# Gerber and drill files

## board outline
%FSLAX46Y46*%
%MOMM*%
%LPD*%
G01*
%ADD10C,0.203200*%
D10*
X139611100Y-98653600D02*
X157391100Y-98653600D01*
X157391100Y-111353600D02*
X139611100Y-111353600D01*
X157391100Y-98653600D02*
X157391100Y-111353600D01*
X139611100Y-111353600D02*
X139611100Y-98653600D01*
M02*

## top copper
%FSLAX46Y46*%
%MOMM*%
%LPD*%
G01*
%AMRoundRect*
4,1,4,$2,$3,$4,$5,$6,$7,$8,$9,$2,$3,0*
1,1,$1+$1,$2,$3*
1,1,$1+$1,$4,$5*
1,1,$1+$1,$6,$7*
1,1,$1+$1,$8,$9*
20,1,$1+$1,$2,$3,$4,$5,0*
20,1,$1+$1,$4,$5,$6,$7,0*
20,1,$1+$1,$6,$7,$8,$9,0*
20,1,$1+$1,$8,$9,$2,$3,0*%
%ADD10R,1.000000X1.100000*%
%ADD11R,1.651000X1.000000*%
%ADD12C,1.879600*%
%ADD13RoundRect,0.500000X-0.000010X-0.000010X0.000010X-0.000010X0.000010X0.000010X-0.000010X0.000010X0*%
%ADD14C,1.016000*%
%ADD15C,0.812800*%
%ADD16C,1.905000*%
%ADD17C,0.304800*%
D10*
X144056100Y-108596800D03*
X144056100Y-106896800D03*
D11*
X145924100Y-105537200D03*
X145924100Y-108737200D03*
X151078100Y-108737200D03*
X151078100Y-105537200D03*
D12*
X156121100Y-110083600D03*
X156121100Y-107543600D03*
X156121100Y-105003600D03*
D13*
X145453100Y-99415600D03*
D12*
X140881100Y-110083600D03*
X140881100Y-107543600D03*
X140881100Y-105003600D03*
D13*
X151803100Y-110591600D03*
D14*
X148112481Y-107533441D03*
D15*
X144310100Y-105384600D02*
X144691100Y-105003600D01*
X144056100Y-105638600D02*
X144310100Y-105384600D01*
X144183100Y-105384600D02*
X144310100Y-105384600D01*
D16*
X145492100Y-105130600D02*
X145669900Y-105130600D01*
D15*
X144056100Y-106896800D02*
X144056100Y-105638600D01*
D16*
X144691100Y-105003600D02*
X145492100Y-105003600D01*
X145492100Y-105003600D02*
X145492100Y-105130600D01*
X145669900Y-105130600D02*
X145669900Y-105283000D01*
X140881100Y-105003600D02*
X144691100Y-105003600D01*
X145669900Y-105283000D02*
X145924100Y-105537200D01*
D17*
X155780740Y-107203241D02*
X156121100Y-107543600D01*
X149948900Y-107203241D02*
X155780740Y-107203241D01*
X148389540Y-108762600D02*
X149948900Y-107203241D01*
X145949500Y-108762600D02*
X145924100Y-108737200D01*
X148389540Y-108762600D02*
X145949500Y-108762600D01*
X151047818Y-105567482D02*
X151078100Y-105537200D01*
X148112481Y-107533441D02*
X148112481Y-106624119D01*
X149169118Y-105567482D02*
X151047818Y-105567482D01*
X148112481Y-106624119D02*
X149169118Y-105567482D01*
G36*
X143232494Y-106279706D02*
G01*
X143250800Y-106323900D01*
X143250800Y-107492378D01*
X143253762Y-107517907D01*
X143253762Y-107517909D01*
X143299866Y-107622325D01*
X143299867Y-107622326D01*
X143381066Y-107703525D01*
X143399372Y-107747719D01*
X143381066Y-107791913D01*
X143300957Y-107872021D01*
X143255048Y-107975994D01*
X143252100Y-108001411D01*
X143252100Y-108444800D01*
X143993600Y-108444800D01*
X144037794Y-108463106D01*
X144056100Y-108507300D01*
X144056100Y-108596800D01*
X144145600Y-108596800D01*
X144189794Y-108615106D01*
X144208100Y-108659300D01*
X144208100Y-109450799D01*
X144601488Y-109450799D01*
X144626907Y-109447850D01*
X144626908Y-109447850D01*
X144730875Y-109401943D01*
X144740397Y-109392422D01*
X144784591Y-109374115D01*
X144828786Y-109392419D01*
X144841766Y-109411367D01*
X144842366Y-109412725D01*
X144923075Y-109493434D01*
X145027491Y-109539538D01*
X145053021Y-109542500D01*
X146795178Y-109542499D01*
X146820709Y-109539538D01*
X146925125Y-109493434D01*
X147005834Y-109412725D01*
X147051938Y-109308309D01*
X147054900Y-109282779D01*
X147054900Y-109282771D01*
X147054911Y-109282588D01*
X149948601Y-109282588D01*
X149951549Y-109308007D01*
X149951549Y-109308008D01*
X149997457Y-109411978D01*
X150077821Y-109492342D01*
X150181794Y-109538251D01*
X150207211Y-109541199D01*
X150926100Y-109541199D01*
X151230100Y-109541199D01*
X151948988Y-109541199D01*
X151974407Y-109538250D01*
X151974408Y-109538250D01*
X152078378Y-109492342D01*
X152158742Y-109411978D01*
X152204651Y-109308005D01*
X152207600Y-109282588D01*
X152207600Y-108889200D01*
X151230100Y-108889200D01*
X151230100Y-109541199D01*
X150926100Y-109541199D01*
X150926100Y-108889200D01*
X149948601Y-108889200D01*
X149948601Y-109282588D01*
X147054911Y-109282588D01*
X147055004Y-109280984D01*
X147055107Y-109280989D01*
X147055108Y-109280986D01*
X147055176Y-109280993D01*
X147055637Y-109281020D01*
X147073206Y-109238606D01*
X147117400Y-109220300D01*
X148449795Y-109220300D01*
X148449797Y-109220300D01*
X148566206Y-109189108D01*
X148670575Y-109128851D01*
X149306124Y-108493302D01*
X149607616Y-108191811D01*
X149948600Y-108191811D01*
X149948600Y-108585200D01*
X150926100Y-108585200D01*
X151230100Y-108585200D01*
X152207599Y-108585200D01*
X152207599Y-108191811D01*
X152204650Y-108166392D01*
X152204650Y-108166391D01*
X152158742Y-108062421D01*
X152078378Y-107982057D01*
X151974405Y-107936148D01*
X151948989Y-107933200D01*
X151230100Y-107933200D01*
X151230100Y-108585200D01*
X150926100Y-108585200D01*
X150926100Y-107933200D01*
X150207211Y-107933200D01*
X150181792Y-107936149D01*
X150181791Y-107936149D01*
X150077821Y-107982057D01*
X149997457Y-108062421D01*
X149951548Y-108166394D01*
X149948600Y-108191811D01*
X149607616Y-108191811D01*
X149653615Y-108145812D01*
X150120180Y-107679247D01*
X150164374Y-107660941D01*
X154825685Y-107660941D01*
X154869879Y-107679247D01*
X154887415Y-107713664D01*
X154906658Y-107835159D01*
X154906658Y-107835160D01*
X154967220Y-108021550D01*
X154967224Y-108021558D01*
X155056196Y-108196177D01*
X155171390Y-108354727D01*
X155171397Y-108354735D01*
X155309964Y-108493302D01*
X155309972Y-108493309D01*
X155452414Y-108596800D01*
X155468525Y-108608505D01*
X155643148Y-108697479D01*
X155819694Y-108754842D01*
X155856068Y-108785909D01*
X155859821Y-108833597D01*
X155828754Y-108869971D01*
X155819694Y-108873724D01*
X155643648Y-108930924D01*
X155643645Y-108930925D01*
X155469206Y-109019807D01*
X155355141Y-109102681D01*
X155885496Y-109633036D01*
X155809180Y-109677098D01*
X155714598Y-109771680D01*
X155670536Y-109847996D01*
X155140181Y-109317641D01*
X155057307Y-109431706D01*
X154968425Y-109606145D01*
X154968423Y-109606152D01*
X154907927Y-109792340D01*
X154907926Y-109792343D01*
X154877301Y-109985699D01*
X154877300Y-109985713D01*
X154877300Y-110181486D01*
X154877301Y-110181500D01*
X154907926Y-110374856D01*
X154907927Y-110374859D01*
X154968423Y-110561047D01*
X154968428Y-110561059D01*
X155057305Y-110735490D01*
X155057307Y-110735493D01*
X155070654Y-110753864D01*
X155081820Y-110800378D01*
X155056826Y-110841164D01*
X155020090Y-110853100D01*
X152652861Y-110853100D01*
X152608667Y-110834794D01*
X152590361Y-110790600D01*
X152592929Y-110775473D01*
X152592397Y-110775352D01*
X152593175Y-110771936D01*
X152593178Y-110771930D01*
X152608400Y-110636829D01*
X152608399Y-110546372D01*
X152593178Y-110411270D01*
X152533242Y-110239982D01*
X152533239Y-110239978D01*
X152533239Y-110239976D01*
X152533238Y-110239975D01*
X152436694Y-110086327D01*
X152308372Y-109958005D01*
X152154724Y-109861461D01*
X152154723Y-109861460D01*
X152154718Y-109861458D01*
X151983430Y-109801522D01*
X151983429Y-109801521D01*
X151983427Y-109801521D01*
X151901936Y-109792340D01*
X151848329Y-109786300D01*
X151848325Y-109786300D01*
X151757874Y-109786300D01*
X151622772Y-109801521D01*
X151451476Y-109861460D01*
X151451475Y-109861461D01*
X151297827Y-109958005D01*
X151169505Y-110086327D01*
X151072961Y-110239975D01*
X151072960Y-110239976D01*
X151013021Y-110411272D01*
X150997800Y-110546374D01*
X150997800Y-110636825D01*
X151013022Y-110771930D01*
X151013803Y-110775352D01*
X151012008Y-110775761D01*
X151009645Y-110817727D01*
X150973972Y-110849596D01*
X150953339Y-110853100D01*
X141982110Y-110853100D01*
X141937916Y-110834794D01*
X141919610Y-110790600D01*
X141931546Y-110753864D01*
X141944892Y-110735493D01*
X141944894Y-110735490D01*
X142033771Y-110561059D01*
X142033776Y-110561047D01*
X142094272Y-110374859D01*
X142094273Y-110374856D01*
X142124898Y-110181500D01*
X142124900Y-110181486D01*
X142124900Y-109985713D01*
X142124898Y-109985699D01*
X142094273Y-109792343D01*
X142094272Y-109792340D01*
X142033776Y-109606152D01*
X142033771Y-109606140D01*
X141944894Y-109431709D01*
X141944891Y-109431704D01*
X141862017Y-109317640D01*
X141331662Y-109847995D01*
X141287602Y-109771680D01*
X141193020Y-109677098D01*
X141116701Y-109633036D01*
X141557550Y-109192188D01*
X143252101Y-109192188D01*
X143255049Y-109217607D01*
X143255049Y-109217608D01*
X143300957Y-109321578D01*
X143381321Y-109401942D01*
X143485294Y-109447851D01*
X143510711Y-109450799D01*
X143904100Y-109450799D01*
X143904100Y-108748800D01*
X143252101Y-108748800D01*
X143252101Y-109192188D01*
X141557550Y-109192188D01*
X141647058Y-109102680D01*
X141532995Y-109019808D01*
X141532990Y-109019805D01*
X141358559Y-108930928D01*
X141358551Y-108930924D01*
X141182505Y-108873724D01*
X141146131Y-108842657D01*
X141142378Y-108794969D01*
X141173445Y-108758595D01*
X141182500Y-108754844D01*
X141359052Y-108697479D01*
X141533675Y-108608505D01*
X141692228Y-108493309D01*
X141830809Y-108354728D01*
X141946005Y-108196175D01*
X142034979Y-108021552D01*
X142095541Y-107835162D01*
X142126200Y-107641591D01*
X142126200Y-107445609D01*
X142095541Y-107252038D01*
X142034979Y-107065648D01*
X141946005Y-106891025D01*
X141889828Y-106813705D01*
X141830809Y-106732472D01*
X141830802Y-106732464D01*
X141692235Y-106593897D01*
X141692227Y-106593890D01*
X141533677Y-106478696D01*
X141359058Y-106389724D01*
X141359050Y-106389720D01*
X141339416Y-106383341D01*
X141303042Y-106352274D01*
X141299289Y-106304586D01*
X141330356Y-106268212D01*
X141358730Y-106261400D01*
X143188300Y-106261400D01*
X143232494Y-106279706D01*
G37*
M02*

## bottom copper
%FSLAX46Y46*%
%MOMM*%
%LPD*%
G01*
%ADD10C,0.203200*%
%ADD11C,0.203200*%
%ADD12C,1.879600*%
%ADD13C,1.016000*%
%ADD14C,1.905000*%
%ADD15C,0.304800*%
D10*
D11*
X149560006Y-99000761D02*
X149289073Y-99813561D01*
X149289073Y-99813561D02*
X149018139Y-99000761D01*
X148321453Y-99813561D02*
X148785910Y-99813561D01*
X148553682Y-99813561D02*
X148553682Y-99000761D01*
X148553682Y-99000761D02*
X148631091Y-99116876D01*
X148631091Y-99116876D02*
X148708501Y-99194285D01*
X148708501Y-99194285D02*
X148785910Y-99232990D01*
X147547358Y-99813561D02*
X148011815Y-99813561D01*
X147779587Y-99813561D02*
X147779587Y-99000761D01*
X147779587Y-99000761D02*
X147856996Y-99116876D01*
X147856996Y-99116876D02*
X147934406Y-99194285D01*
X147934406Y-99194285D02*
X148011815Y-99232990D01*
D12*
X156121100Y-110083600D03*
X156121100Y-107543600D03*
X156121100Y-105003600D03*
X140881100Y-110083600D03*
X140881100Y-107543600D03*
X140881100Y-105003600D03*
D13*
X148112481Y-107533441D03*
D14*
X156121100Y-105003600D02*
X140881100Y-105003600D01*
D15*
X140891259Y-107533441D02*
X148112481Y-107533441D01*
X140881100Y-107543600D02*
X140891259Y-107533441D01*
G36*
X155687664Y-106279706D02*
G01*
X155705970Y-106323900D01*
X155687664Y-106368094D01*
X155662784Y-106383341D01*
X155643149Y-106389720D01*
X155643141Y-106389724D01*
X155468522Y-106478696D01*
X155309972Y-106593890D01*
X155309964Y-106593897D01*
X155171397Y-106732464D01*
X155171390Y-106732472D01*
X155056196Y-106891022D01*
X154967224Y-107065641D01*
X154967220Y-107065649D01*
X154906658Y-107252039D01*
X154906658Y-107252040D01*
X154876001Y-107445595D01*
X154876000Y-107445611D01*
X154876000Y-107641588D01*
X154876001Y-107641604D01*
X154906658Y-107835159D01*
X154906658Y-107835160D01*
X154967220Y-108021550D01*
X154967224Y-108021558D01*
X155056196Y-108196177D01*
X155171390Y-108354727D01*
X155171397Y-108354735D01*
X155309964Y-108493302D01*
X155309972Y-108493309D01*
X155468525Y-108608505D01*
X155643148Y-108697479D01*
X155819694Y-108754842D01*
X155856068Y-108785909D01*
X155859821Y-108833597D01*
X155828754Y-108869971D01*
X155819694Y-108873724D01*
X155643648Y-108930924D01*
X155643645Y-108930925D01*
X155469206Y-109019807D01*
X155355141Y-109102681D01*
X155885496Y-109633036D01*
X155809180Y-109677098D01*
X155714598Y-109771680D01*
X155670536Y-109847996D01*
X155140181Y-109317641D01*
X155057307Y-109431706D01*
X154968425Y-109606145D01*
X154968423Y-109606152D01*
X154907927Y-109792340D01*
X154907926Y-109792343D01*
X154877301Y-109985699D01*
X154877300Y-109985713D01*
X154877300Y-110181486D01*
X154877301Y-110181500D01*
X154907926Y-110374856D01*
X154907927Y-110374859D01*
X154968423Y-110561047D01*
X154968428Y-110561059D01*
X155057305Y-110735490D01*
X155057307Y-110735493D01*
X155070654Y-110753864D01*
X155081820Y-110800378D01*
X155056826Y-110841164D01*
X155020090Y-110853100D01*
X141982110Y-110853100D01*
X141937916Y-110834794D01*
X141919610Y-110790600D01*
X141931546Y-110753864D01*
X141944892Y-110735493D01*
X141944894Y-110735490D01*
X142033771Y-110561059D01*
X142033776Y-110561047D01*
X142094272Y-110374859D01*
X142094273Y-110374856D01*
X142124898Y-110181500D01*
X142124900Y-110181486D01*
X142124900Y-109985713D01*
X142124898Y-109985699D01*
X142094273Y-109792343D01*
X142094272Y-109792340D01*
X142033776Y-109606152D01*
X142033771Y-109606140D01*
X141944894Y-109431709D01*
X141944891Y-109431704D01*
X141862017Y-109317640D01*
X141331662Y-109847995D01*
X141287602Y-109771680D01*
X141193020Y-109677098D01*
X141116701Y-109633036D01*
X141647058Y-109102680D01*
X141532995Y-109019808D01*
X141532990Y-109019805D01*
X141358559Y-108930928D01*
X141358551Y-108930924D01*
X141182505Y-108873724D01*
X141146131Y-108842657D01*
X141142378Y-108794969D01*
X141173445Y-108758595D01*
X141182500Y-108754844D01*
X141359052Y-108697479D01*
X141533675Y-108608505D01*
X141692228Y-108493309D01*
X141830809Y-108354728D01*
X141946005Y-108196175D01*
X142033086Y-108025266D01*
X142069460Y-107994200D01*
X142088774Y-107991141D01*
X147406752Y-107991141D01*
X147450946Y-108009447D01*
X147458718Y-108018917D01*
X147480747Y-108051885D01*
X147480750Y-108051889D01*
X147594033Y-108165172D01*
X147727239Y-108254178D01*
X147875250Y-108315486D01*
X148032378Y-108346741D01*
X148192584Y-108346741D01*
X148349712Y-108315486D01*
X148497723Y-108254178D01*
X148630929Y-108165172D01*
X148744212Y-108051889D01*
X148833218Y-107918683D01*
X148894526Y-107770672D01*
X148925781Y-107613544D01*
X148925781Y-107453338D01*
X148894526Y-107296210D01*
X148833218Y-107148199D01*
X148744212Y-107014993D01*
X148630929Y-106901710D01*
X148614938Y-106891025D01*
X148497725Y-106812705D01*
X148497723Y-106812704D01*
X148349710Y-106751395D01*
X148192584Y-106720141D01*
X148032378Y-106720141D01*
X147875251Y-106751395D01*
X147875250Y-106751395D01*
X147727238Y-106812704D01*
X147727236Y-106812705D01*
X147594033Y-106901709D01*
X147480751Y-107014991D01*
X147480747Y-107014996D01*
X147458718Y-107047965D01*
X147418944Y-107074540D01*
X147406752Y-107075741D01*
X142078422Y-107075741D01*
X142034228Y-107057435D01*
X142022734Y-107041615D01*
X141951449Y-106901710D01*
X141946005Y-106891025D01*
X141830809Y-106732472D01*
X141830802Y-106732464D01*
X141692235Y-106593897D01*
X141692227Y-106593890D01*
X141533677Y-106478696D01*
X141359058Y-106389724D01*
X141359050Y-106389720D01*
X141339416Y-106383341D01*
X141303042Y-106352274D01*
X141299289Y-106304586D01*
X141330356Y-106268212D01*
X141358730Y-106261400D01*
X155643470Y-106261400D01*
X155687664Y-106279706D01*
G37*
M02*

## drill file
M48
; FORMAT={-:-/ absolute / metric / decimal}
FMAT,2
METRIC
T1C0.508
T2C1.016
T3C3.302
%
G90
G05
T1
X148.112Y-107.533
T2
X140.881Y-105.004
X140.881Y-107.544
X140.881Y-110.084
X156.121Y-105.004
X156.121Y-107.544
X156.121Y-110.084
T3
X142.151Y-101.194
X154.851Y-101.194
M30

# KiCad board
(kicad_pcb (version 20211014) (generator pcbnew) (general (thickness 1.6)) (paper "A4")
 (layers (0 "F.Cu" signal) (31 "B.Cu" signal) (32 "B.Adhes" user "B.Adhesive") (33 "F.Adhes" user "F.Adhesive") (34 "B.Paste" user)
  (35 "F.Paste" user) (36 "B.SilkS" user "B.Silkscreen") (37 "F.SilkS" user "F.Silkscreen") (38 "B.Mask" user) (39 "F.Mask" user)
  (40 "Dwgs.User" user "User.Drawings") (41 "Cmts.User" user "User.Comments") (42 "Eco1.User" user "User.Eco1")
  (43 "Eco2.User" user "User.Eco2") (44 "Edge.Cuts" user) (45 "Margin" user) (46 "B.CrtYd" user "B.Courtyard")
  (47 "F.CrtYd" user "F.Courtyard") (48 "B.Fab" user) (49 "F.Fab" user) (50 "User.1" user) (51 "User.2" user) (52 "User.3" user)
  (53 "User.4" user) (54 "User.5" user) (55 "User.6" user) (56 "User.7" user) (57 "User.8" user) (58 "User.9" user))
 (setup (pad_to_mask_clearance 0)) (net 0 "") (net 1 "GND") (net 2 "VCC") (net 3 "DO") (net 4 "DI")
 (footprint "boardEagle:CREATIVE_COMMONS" (layer "F.Cu") (at 118.159513 124.0536)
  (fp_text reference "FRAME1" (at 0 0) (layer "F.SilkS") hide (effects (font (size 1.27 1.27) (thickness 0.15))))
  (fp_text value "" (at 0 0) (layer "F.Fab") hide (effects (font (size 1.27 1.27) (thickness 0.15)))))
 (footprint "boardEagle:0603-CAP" (layer "F.Cu") (at 144.0561 107.7468 90)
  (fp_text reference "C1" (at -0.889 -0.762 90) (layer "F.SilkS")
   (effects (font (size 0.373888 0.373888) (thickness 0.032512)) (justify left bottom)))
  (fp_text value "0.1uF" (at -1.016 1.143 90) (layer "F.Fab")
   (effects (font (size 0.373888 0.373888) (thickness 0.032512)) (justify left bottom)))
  (pad "1" smd rect (at -0.85 0 90) (size 1.1 1) (layers "F.Cu" "F.Paste" "F.Mask") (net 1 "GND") (solder_mask_margin 0.1016))
  (pad "2" smd rect (at 0.85 0 90) (size 1.1 1) (layers "F.Cu" "F.Paste" "F.Mask") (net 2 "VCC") (solder_mask_margin 0.1016)))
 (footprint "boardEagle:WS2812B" (layer "F.Cu") (at 148.5011 107.1372)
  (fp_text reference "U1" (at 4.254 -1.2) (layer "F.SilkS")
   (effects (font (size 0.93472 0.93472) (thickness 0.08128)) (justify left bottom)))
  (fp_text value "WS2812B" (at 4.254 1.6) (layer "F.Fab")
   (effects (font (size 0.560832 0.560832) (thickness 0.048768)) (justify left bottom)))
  (pad "1" smd rect (at -2.577 -1.6) (size 1.651 1) (layers "F.Cu" "F.Paste" "F.Mask") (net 2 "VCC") (solder_mask_margin 0.1016))
  (pad "2" smd rect (at -2.577 1.6) (size 1.651 1) (layers "F.Cu" "F.Paste" "F.Mask") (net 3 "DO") (solder_mask_margin 0.1016))
  (pad "3" smd rect (at 2.577 1.6) (size 1.651 1) (layers "F.Cu" "F.Paste" "F.Mask") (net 1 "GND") (solder_mask_margin 0.1016))
  (pad "4" smd rect (at 2.577 -1.6) (size 1.651 1) (layers "F.Cu" "F.Paste" "F.Mask") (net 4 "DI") (solder_mask_margin 0.1016)))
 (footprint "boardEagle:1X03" (layer "F.Cu") (at 156.1211 110.0836 90)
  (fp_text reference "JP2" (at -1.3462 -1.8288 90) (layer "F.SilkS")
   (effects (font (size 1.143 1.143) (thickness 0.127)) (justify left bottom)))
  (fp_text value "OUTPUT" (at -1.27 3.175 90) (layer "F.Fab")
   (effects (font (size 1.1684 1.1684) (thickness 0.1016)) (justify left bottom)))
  (pad "1" thru_hole circle (at 0 0 180) (size 1.8796 1.8796) (drill 1.016) (layers *.Cu *.Mask) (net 1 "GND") (solder_mask_margin 0.1016))
  (pad "2" thru_hole circle (at 2.54 0 180) (size 1.8796 1.8796) (drill 1.016) (layers *.Cu *.Mask) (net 3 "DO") (solder_mask_margin 0.1016))
  (pad "3" thru_hole circle (at 5.08 0 180) (size 1.8796 1.8796) (drill 1.016) (layers *.Cu *.Mask) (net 2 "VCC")
   (solder_mask_margin 0.1016)))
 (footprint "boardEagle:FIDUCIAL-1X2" (layer "F.Cu") (at 145.4531 99.4156)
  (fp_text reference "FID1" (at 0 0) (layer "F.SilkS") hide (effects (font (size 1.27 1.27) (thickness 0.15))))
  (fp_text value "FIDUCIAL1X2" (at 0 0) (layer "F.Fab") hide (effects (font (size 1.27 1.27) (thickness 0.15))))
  (pad "1" smd roundrect (at 0 0) (size 1 1) (layers "F.Cu" "F.Mask") (roundrect_rratio 0.5) (solder_mask_margin 0.1016)))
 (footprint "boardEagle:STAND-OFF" (layer "F.Cu") (at 142.1511 101.1936)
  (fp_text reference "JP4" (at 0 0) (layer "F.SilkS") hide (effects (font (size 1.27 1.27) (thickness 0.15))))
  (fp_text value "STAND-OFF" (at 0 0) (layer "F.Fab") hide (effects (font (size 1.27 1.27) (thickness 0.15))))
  (pad "" np_thru_hole circle (at 0 0) (size 3.302 3.302) (drill 3.302) (layers *.Cu *.Mask)))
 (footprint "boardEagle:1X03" (layer "F.Cu") (at 140.8811 110.0836 90)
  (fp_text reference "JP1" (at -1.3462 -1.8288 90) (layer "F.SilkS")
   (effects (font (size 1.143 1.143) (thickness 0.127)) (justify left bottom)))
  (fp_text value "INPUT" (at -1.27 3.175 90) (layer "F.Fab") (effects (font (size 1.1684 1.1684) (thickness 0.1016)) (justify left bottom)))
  (pad "1" thru_hole circle (at 0 0 180) (size 1.8796 1.8796) (drill 1.016) (layers *.Cu *.Mask) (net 1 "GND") (solder_mask_margin 0.1016))
  (pad "2" thru_hole circle (at 2.54 0 180) (size 1.8796 1.8796) (drill 1.016) (layers *.Cu *.Mask) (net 4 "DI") (solder_mask_margin 0.1016))
  (pad "3" thru_hole circle (at 5.08 0 180) (size 1.8796 1.8796) (drill 1.016) (layers *.Cu *.Mask) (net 2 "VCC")
   (solder_mask_margin 0.1016)))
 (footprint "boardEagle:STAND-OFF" (layer "F.Cu") (at 154.8511 101.1936)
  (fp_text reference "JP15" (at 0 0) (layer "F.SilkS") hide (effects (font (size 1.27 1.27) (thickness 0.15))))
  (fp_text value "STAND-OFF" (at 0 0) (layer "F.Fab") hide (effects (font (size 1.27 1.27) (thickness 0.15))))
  (pad "" np_thru_hole circle (at 0 0) (size 3.302 3.302) (drill 3.302) (layers *.Cu *.Mask)))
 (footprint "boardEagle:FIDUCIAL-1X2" (layer "F.Cu") (at 151.8031 110.5916)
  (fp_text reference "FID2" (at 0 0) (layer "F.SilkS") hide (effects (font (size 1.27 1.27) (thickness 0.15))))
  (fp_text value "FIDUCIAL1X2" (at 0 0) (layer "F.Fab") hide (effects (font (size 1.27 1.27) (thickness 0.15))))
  (pad "1" smd roundrect (at 0 0) (size 1 1) (layers "F.Cu" "F.Mask") (roundrect_rratio 0.5) (solder_mask_margin 0.1016)))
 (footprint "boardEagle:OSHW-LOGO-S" (layer "B.Cu") (at 148.587459 102.217222 180)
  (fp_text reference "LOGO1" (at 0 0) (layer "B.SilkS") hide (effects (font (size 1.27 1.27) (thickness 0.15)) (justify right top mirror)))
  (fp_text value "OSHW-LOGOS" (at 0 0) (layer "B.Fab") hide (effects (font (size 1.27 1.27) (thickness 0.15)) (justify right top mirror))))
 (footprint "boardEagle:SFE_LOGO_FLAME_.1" (layer "B.Cu") (at 149.768559 106.913679 180)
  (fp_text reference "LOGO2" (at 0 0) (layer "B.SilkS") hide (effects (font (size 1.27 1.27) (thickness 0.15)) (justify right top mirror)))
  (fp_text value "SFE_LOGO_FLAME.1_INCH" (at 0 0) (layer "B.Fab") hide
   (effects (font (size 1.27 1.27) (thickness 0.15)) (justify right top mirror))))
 (gr_line (start 139.6111 98.6536) (end 157.3911 98.6536) (layer "Edge.Cuts") (width 0.2032))
 (gr_line (start 157.3911 111.3536) (end 139.6111 111.3536) (layer "Edge.Cuts") (width 0.2032))
 (gr_line (start 157.3911 98.6536) (end 157.3911 111.3536) (layer "Edge.Cuts") (width 0.2032))
 (gr_line (start 139.6111 111.3536) (end 139.6111 98.6536) (layer "Edge.Cuts") (width 0.2032))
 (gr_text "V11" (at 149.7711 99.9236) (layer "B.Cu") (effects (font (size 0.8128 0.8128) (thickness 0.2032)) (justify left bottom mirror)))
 (segment (start 144.3101 105.3846) (end 144.6911 105.0036) (width 0.8128) (layer "F.Cu") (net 2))
 (segment (start 144.0561 105.6386) (end 144.3101 105.3846) (width 0.8128) (layer "F.Cu") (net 2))
 (segment (start 144.1831 105.3846) (end 144.3101 105.3846) (width 0.8128) (layer "F.Cu") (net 2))
 (segment (start 145.4921 105.1306) (end 145.6699 105.1306) (width 1.905) (layer "F.Cu") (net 2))
 (segment (start 144.0561 106.8968) (end 144.0561 105.6386) (width 0.8128) (layer "F.Cu") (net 2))
 (segment (start 144.6911 105.0036) (end 145.4921 105.0036) (width 1.905) (layer "F.Cu") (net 2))
 (segment (start 145.4921 105.0036) (end 145.4921 105.1306) (width 1.905) (layer "F.Cu") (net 2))
 (segment (start 145.6699 105.1306) (end 145.6699 105.283) (width 1.905) (layer "F.Cu") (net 2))
 (segment (start 140.8811 105.0036) (end 144.6911 105.0036) (width 1.905) (layer "F.Cu") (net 2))
 (segment (start 145.6699 105.283) (end 145.9241 105.5372) (width 1.905) (layer "F.Cu") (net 2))
 (segment (start 156.1211 105.0036) (end 140.8811 105.0036) (width 1.905) (layer "B.Cu") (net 2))
 (segment (start 155.78074 107.203241) (end 156.1211 107.5436) (width 0.3048) (layer "F.Cu") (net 3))
 (segment (start 149.9489 107.203241) (end 155.78074 107.203241) (width 0.3048) (layer "F.Cu") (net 3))
 (segment (start 148.38954 108.7626) (end 149.9489 107.203241) (width 0.3048) (layer "F.Cu") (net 3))
 (segment (start 145.9495 108.7626) (end 145.9241 108.7372) (width 0.3048) (layer "F.Cu") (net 3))
 (segment (start 148.38954 108.7626) (end 145.9495 108.7626) (width 0.3048) (layer "F.Cu") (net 3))
 (segment (start 151.047818 105.567482) (end 151.0781 105.5372) (width 0.3048) (layer "F.Cu") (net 4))
 (segment (start 148.112481 107.533441) (end 148.112481 106.624119) (width 0.3048) (layer "F.Cu") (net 4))
 (segment (start 149.169118 105.567482) (end 151.047818 105.567482) (width 0.3048) (layer "F.Cu") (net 4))
 (segment (start 148.112481 106.624119) (end 149.169118 105.567482) (width 0.3048) (layer "F.Cu") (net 4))
 (via (at 148.112481 107.533441) (size 1.016) (drill 0.508) (layers "F.Cu" "B.Cu") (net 4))
 (segment (start 140.891259 107.533441) (end 148.112481 107.533441) (width 0.3048) (layer "B.Cu") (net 4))
 (segment (start 140.8811 107.5436) (end 140.891259 107.533441) (width 0.3048) (layer "B.Cu") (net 4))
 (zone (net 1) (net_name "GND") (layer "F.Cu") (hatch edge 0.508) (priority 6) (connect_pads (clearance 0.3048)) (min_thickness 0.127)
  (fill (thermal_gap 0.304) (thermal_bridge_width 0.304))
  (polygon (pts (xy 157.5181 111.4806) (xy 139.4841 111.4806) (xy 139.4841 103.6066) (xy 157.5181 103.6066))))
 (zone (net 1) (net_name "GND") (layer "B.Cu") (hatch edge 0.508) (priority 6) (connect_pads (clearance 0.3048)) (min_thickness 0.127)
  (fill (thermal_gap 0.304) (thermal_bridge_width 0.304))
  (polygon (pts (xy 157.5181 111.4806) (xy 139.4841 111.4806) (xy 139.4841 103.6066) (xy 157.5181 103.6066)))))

